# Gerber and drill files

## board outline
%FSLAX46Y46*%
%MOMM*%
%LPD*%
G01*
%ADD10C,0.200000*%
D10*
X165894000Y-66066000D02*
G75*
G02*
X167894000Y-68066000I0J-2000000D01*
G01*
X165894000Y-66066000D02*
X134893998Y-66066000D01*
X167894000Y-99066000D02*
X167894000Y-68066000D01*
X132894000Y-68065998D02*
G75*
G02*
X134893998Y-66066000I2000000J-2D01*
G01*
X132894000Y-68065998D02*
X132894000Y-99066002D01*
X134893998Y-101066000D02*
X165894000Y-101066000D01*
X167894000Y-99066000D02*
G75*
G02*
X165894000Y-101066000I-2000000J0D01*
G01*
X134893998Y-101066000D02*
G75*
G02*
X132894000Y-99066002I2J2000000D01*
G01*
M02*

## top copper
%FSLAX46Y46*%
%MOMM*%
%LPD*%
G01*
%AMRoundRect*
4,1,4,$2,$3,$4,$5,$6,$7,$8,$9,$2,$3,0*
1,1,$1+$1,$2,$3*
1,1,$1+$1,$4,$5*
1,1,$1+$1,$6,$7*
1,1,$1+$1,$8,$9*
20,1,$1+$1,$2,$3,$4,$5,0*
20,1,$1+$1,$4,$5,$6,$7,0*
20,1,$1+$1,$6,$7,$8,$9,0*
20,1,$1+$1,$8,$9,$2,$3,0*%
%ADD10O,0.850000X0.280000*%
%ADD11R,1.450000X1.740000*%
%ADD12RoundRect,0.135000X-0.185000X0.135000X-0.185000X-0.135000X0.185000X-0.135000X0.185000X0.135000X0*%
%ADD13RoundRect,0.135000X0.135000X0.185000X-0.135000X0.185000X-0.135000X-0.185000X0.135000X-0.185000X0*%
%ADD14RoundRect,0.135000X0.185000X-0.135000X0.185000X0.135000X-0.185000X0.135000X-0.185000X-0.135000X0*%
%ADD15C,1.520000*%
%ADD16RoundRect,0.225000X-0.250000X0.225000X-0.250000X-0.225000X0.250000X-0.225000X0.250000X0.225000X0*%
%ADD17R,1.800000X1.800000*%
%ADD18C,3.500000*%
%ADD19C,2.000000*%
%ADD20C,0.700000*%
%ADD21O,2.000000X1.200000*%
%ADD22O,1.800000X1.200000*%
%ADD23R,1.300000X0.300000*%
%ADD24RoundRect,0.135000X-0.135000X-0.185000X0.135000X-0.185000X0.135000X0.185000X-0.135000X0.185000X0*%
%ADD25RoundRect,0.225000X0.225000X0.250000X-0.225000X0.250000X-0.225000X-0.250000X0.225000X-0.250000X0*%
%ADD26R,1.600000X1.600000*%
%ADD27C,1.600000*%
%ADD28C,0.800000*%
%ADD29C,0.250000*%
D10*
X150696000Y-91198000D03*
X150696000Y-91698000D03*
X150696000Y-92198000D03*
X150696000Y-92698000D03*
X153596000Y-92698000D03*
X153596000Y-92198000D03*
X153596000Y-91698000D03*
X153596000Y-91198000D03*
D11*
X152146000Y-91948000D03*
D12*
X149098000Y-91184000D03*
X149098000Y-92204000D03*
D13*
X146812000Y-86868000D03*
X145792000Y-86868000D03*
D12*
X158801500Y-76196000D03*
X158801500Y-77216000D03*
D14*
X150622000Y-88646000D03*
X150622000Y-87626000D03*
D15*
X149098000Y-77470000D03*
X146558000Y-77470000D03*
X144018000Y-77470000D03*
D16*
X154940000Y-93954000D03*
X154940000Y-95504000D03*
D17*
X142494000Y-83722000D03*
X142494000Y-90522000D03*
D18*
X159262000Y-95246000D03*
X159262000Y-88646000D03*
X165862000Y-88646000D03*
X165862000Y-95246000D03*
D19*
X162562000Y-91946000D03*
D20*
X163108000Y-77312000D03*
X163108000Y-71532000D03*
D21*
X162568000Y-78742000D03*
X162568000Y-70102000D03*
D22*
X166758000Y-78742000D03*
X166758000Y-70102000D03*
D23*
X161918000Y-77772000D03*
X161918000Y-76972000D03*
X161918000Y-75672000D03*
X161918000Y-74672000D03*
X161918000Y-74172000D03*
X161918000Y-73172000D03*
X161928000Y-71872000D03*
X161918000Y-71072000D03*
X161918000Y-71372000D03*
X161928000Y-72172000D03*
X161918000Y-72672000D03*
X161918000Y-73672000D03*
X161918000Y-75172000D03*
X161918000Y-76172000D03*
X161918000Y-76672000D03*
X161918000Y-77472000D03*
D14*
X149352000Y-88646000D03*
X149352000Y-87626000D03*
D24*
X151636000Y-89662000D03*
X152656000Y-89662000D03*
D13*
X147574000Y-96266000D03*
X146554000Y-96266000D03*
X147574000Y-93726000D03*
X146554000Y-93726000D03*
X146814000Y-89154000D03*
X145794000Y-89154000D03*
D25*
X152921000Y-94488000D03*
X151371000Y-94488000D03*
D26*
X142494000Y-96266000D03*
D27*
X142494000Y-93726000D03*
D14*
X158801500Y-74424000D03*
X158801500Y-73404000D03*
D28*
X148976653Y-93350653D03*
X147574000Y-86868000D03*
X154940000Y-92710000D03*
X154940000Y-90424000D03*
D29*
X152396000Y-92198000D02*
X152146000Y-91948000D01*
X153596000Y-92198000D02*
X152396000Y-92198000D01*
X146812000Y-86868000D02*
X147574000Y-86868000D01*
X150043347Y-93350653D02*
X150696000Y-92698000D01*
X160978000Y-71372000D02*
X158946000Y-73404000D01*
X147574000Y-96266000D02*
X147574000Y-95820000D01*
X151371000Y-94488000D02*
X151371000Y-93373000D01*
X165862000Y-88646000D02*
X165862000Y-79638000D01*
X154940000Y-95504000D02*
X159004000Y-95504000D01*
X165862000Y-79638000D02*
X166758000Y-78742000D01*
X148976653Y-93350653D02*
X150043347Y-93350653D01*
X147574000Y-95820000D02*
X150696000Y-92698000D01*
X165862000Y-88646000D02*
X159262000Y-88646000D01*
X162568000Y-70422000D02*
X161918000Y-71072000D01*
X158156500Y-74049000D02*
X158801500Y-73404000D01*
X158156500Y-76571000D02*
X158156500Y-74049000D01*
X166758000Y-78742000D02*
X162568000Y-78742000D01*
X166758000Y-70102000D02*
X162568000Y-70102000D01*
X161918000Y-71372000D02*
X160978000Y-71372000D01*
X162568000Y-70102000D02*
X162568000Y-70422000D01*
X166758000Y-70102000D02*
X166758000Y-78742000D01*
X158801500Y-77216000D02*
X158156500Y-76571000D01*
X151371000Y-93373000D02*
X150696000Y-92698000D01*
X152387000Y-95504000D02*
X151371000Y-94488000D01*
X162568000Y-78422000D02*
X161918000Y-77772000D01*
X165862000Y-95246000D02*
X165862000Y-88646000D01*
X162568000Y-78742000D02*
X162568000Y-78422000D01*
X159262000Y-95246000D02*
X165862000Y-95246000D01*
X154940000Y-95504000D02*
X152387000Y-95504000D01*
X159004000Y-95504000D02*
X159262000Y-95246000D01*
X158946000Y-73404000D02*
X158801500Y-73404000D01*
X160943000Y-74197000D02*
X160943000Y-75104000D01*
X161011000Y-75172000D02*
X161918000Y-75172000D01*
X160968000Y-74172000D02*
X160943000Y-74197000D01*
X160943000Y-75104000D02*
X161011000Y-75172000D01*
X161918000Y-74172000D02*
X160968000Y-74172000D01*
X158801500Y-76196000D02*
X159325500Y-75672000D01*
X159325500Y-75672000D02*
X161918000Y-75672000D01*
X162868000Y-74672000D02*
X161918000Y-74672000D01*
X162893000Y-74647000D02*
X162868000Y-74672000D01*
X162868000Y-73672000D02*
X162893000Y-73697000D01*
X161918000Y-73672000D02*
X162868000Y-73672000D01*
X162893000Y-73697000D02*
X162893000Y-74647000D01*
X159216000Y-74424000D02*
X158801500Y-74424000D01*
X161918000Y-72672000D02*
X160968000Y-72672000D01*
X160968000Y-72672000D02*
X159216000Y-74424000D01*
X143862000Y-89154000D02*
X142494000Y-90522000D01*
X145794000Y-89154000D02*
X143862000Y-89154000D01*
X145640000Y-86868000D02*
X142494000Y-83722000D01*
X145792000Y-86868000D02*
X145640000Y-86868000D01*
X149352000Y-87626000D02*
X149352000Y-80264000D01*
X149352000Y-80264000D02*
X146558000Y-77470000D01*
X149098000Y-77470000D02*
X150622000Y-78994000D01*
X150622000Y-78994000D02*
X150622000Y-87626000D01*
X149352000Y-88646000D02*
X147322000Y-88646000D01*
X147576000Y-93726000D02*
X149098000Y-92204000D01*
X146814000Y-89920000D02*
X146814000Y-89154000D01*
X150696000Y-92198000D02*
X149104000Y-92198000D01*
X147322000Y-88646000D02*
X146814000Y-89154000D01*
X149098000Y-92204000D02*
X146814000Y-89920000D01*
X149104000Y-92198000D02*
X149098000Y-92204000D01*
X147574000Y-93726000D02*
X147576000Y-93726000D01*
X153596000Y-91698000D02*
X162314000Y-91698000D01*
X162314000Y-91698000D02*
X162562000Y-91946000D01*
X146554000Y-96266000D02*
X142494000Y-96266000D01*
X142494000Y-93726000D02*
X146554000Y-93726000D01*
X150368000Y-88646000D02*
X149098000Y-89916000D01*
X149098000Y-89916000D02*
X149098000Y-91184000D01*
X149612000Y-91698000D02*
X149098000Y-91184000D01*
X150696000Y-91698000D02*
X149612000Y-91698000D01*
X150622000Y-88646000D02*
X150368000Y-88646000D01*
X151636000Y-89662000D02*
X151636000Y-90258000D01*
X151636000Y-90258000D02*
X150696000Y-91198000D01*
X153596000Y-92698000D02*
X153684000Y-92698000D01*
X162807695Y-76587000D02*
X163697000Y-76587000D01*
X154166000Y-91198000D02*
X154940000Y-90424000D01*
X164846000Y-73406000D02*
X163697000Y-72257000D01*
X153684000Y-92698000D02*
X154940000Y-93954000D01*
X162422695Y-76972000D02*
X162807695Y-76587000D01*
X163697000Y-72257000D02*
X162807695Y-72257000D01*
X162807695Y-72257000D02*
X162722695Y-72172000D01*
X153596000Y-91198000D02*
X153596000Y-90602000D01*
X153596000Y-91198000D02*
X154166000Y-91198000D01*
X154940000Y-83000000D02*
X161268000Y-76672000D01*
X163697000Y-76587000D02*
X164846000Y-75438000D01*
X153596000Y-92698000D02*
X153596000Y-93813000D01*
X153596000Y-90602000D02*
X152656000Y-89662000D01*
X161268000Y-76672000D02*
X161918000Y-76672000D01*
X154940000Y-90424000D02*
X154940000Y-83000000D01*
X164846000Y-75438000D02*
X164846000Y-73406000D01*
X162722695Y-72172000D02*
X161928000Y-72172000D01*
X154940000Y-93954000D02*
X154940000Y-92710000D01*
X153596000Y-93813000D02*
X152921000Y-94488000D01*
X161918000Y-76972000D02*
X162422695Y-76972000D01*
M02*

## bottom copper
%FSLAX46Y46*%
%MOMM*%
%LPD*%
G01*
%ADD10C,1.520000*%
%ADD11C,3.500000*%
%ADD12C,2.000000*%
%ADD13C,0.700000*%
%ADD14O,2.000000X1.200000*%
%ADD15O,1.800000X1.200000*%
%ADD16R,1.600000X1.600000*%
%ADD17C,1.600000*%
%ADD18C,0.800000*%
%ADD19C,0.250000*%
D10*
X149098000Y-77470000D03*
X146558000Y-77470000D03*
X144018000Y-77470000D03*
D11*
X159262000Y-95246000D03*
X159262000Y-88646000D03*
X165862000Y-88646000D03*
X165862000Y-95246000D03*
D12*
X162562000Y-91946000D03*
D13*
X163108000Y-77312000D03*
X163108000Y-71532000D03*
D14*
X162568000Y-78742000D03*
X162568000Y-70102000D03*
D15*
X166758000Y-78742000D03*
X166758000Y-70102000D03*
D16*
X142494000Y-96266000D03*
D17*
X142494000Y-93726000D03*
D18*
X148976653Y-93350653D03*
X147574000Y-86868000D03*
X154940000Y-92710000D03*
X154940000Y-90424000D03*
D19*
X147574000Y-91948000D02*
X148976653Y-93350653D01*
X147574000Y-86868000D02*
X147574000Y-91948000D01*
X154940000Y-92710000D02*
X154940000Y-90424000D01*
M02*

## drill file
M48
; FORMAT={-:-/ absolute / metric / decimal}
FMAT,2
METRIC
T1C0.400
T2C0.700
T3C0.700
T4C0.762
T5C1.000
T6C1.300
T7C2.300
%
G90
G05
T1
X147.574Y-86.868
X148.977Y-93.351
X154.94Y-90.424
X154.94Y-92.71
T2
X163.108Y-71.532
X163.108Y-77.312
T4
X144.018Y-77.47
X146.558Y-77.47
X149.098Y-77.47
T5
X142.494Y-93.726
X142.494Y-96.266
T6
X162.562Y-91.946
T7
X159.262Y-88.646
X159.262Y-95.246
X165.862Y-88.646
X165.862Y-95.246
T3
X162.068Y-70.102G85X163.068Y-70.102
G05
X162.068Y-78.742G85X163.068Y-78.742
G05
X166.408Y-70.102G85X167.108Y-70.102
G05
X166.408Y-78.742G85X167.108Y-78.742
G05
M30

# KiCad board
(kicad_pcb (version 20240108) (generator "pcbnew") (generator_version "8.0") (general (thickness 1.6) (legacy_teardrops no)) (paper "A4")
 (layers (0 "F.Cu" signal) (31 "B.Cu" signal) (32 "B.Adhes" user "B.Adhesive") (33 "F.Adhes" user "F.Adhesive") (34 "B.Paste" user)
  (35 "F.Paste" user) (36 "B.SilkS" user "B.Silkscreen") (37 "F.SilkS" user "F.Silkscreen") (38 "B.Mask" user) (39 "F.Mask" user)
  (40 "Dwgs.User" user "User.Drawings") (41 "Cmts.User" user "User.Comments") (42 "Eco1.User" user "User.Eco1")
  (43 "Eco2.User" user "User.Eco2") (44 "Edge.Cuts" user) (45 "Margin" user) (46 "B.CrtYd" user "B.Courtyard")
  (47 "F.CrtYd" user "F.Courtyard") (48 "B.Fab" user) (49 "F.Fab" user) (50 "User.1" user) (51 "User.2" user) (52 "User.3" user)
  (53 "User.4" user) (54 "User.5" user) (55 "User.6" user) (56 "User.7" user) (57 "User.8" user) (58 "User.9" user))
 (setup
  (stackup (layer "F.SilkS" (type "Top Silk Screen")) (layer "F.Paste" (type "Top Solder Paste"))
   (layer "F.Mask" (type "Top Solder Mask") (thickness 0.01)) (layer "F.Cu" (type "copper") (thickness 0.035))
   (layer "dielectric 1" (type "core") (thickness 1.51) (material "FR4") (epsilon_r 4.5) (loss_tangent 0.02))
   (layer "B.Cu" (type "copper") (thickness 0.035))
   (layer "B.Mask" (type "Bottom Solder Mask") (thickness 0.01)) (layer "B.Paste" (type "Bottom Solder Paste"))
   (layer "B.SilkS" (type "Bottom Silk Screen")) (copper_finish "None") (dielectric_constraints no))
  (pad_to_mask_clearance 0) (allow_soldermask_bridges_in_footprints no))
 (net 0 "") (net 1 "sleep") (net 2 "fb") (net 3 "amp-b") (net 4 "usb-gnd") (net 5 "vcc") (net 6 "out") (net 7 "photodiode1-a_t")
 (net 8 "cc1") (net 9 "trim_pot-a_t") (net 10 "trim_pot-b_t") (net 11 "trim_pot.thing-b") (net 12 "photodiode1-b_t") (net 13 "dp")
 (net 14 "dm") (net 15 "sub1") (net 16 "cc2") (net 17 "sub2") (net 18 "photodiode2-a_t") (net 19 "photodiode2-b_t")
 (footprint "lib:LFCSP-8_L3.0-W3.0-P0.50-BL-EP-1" (layer "F.Cu") (at 152.146 91.948 -90)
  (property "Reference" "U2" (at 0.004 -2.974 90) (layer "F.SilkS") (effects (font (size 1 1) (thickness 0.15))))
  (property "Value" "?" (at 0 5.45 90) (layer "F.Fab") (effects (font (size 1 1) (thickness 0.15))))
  (pad "1" smd oval (at -0.75 1.45 90) (size 0.28 0.85) (layers "F.Cu" "F.Paste" "F.Mask") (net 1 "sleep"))
  (pad "2" smd oval (at -0.25 1.45 90) (size 0.28 0.85) (layers "F.Cu" "F.Paste" "F.Mask") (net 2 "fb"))
  (pad "3" smd oval (at 0.25 1.45 90) (size 0.28 0.85) (layers "F.Cu" "F.Paste" "F.Mask") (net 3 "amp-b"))
  (pad "4" smd oval (at 0.75 1.45 90) (size 0.28 0.85) (layers "F.Cu" "F.Paste" "F.Mask") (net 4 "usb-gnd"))
  (pad "5" smd oval (at 0.75 -1.45 90) (size 0.28 0.85) (layers "F.Cu" "F.Paste" "F.Mask") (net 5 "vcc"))
  (pad "6" smd oval (at 0.25 -1.45 90) (size 0.28 0.85) (layers "F.Cu" "F.Paste" "F.Mask"))
  (pad "7" smd oval (at -0.25 -1.45 90) (size 0.28 0.85) (layers "F.Cu" "F.Paste" "F.Mask") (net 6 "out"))
  (pad "8" smd oval (at -0.75 -1.45 90) (size 0.28 0.85) (layers "F.Cu" "F.Paste" "F.Mask") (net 5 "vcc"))
  (pad "9" smd rect (at 0 0 270) (size 1.74 1.45) (layers "F.Cu" "F.Paste" "F.Mask")))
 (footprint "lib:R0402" (layer "F.Cu") (at 149.098 91.694 -90)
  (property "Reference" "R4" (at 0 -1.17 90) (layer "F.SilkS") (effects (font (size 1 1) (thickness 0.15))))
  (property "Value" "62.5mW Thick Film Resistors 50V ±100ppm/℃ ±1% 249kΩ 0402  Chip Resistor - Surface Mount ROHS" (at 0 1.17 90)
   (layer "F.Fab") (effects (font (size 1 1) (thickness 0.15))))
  (pad "1" smd roundrect (at -0.51 0 270) (size 0.54 0.64) (layers "F.Cu" "F.Paste" "F.Mask") (roundrect_rratio 0.25) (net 2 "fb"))
  (pad "2" smd roundrect (at 0.51 0 270) (size 0.54 0.64) (layers "F.Cu" "F.Paste" "F.Mask") (roundrect_rratio 0.25) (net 3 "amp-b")))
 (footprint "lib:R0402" (layer "F.Cu") (at 146.302 86.868 180)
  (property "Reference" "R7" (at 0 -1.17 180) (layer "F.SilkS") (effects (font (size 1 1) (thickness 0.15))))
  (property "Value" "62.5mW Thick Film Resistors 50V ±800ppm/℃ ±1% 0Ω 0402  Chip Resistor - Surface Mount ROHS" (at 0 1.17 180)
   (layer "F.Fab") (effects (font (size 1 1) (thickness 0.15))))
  (pad "1" smd roundrect (at -0.51 0 180) (size 0.54 0.64) (layers "F.Cu" "F.Paste" "F.Mask") (roundrect_rratio 0.25) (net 4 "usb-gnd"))
  (pad "2" smd roundrect (at 0.51 0 180) (size 0.54 0.64) (layers "F.Cu" "F.Paste" "F.Mask") (roundrect_rratio 0.25)
   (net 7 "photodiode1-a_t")))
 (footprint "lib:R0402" (layer "F.Cu") (at 158.8015 76.706 -90)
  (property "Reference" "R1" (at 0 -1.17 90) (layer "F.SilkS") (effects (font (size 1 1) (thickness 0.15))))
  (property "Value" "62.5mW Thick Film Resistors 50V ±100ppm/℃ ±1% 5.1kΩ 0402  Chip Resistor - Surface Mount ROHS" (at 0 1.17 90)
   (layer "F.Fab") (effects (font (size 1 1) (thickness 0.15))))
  (pad "1" smd roundrect (at -0.51 0 270) (size 0.54 0.64) (layers "F.Cu" "F.Paste" "F.Mask") (roundrect_rratio 0.25) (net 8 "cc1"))
  (pad "2" smd roundrect (at 0.51 0 270) (size 0.54 0.64) (layers "F.Cu" "F.Paste" "F.Mask") (roundrect_rratio 0.25) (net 4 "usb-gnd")))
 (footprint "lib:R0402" (layer "F.Cu") (at 150.622 88.136 90)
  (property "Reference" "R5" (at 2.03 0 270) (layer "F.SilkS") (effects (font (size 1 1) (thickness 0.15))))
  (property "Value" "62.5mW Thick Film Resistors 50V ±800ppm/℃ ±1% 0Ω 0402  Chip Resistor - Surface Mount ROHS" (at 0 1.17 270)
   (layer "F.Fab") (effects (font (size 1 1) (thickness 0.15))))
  (pad "1" smd roundrect (at -0.51 0 90) (size 0.54 0.64) (layers "F.Cu" "F.Paste" "F.Mask") (roundrect_rratio 0.25) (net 2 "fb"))
  (pad "2" smd roundrect (at 0.51 0 90) (size 0.54 0.64) (layers "F.Cu" "F.Paste" "F.Mask") (roundrect_rratio 0.25) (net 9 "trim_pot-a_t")))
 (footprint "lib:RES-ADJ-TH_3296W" (layer "F.Cu") (at 146.558 77.47 -90)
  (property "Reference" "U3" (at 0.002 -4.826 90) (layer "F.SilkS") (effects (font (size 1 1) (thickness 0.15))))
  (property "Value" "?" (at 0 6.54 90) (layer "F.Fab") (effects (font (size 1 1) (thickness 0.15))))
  (pad "1" thru_hole circle (at 0 -2.54 180) (size 1.52 1.52) (drill 0.762) (layers "*.Cu" "*.Mask") (remove_unused_layers no)
   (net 9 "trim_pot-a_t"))
  (pad "2" thru_hole circle (at 0 0 180) (size 1.52 1.52) (drill 0.762) (layers "*.Cu" "*.Mask") (remove_unused_layers no)
   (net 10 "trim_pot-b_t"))
  (pad "3" thru_hole circle (at 0 2.54 180) (size 1.52 1.52) (drill 0.762) (layers "*.Cu" "*.Mask") (remove_unused_layers no)
   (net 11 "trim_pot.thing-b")))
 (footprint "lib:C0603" (layer "F.Cu") (at 154.94 94.729 -90)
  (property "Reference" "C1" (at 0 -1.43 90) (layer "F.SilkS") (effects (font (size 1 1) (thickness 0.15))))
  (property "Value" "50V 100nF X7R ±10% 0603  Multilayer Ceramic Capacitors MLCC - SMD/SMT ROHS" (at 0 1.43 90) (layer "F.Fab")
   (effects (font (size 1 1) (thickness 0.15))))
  (pad "1" smd roundrect (at -0.775 0 270) (size 0.9 0.95) (layers "F.Cu" "F.Paste" "F.Mask") (roundrect_rratio 0.25) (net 5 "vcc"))
  (pad "2" smd roundrect (at 0.775 0 270) (size 0.9 0.95) (layers "F.Cu" "F.Paste" "F.Mask") (roundrect_rratio 0.25) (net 4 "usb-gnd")))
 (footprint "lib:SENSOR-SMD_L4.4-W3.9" (layer "F.Cu") (at 142.494 87.122 -90)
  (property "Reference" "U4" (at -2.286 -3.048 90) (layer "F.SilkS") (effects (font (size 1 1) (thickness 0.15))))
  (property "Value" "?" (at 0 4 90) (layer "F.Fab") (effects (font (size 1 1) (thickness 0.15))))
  (pad "1" smd rect (at -3.4 0 270) (size 1.8 1.8) (layers "F.Cu" "F.Paste" "F.Mask") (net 7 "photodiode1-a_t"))
  (pad "2" smd rect (at 3.4 0 270) (size 1.8 1.8) (layers "F.Cu" "F.Paste" "F.Mask") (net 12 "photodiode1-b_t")))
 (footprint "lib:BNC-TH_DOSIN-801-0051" (layer "F.Cu") (at 162.562 91.946)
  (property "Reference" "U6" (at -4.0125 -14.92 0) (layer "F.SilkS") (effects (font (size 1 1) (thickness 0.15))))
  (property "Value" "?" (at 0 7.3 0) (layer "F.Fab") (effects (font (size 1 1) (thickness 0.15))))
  (pad "1" thru_hole circle (at -3.3 3.3) (size 3.5 3.5) (drill 2.300021) (layers "*.Cu" "*.Mask") (remove_unused_layers no)
   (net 4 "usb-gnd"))
  (pad "2" thru_hole circle (at -3.3 -3.3) (size 3.5 3.5) (drill 2.300021) (layers "*.Cu" "*.Mask") (remove_unused_layers no)
   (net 4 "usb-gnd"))
  (pad "3" thru_hole circle (at 3.3 -3.3) (size 3.5 3.5) (drill 2.300021) (layers "*.Cu" "*.Mask") (remove_unused_layers no)
   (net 4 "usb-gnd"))
  (pad "4" thru_hole circle (at 3.3 3.3) (size 3.5 3.5) (drill 2.300021) (layers "*.Cu" "*.Mask") (remove_unused_layers no)
   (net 4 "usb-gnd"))
  (pad "5" thru_hole circle (at 0 0) (size 2 2) (drill 1.300023) (layers "*.Cu" "*.Mask") (remove_unused_layers no) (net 6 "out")))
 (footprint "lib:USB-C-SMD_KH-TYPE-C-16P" (layer "F.Cu") (at 164.338 74.422 90)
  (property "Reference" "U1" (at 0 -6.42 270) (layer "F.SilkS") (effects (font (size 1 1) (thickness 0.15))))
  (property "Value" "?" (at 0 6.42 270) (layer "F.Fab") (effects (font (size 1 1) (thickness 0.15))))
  (pad "" thru_hole circle (at -2.89 -1.23 90) (size 0.7 0.7) (drill 0.7) (layers "*.Cu" "*.Mask") (remove_unused_layers no))
  (pad "" thru_hole circle (at 2.89 -1.23 90) (size 0.7 0.7) (drill 0.7) (layers "*.Cu" "*.Mask") (remove_unused_layers no))
  (pad "1" thru_hole oval (at -4.32 -1.77 90) (size 1.2 2) (drill oval 0.700024 1.699997) (layers "*.Cu" "*.Mask") (remove_unused_layers no)
   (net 4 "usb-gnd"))
  (pad "2" thru_hole oval (at 4.32 -1.77 90) (size 1.2 2) (drill oval 0.700024 1.699997) (layers "*.Cu" "*.Mask") (remove_unused_layers no)
   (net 4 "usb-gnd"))
  (pad "3" thru_hole oval (at -4.32 2.42 90) (size 1.2 1.8) (drill oval 0.700024 1.399997) (layers "*.Cu" "*.Mask")
   (remove_unused_layers no) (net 4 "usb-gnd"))
  (pad "4" thru_hole oval (at 4.32 2.42 90) (size 1.2 1.8) (drill oval 0.700024 1.399997) (layers "*.Cu" "*.Mask") (remove_unused_layers no)
   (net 4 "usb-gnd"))
  (pad "A1" smd rect (at -3.35 -2.42 90) (size 0.3 1.3) (layers "F.Cu" "F.Paste" "F.Mask") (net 4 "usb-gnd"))
  (pad "A4" smd rect (at -2.55 -2.42 90) (size 0.3 1.3) (layers "F.Cu" "F.Paste" "F.Mask") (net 5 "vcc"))
  (pad "A5" smd rect (at -1.25 -2.42 90) (size 0.3 1.3) (layers "F.Cu" "F.Paste" "F.Mask") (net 8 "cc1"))
  (pad "A6" smd rect (at -0.25 -2.42 90) (size 0.3 1.3) (layers "F.Cu" "F.Paste" "F.Mask") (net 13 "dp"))
  (pad "A7" smd rect (at 0.25 -2.42 90) (size 0.3 1.3) (layers "F.Cu" "F.Paste" "F.Mask") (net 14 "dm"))
  (pad "A8" smd rect (at 1.25 -2.42 90) (size 0.3 1.3) (layers "F.Cu" "F.Paste" "F.Mask") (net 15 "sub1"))
  (pad "A9" smd rect (at 2.55 -2.41 90) (size 0.3 1.3) (layers "F.Cu" "F.Paste" "F.Mask") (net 5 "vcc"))
  (pad "A12" smd rect (at 3.35 -2.42 90) (size 0.3 1.3) (layers "F.Cu" "F.Paste" "F.Mask") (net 4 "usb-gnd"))
  (pad "B1" smd rect (at 3.05 -2.42 90) (size 0.3 1.3) (layers "F.Cu" "F.Paste" "F.Mask") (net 4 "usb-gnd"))
  (pad "B4" smd rect (at 2.25 -2.41 90) (size 0.3 1.3) (layers "F.Cu" "F.Paste" "F.Mask") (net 5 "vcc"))
  (pad "B5" smd rect (at 1.75 -2.42 90) (size 0.3 1.3) (layers "F.Cu" "F.Paste" "F.Mask") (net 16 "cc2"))
  (pad "B6" smd rect (at 0.75 -2.42 90) (size 0.3 1.3) (layers "F.Cu" "F.Paste" "F.Mask") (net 13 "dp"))
  (pad "B7" smd rect (at -0.75 -2.42 90) (size 0.3 1.3) (layers "F.Cu" "F.Paste" "F.Mask") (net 14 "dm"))
  (pad "B8" smd rect (at -1.75 -2.42 90) (size 0.3 1.3) (layers "F.Cu" "F.Paste" "F.Mask") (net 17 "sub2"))
  (pad "B9" smd rect (at -2.25 -2.42 90) (size 0.3 1.3) (layers "F.Cu" "F.Paste" "F.Mask") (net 5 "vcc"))
  (pad "B12" smd rect (at -3.05 -2.42 90) (size 0.3 1.3) (layers "F.Cu" "F.Paste" "F.Mask") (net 4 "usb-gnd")))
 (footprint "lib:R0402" (layer "F.Cu") (at 149.352 88.136 90)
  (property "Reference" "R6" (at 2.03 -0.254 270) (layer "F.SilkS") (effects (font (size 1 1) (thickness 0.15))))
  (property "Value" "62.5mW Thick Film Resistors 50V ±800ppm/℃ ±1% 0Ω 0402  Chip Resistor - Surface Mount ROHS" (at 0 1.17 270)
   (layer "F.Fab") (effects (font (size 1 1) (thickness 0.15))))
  (pad "1" smd roundrect (at -0.51 0 90) (size 0.54 0.64) (layers "F.Cu" "F.Paste" "F.Mask") (roundrect_rratio 0.25) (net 3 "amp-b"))
  (pad "2" smd roundrect (at 0.51 0 90) (size 0.54 0.64) (layers "F.Cu" "F.Paste" "F.Mask") (roundrect_rratio 0.25) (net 10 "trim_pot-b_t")))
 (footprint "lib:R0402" (layer "F.Cu") (at 152.146 89.662)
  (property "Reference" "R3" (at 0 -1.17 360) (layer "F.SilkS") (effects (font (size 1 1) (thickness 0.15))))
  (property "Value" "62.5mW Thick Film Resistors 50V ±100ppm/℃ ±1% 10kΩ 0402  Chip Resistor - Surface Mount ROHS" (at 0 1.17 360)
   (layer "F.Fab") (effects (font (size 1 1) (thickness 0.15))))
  (pad "1" smd roundrect (at -0.51 0) (size 0.54 0.64) (layers "F.Cu" "F.Paste" "F.Mask") (roundrect_rratio 0.25) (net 1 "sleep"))
  (pad "2" smd roundrect (at 0.51 0) (size 0.54 0.64) (layers "F.Cu" "F.Paste" "F.Mask") (roundrect_rratio 0.25) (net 5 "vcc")))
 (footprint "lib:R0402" (layer "F.Cu") (at 147.064 96.266 180)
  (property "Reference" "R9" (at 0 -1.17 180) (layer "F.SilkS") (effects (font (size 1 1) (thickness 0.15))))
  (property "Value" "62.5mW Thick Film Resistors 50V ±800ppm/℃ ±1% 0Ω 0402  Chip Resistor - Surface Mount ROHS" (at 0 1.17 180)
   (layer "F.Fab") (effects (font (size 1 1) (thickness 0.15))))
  (pad "1" smd roundrect (at -0.51 0 180) (size 0.54 0.64) (layers "F.Cu" "F.Paste" "F.Mask") (roundrect_rratio 0.25) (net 4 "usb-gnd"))
  (pad "2" smd roundrect (at 0.51 0 180) (size 0.54 0.64) (layers "F.Cu" "F.Paste" "F.Mask") (roundrect_rratio 0.25)
   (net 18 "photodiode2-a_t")))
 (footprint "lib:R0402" (layer "F.Cu") (at 147.064 93.726 180)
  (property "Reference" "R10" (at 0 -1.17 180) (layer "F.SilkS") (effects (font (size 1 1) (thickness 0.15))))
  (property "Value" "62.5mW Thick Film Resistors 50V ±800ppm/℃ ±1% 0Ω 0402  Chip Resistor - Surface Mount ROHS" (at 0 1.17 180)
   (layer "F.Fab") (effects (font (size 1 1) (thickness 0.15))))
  (pad "1" smd roundrect (at -0.51 0 180) (size 0.54 0.64) (layers "F.Cu" "F.Paste" "F.Mask") (roundrect_rratio 0.25) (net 3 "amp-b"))
  (pad "2" smd roundrect (at 0.51 0 180) (size 0.54 0.64) (layers "F.Cu" "F.Paste" "F.Mask") (roundrect_rratio 0.25)
   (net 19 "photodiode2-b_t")))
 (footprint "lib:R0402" (layer "F.Cu") (at 146.304 89.154 180)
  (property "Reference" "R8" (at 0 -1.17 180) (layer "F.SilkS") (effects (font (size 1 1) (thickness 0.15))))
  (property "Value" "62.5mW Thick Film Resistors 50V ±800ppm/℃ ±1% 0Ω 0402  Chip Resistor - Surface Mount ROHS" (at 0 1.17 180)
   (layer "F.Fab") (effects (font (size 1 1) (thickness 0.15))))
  (pad "1" smd roundrect (at -0.51 0 180) (size 0.54 0.64) (layers "F.Cu" "F.Paste" "F.Mask") (roundrect_rratio 0.25) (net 3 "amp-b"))
  (pad "2" smd roundrect (at 0.51 0 180) (size 0.54 0.64) (layers "F.Cu" "F.Paste" "F.Mask") (roundrect_rratio 0.25)
   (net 12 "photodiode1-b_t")))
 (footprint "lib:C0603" (layer "F.Cu") (at 152.146 94.488 180)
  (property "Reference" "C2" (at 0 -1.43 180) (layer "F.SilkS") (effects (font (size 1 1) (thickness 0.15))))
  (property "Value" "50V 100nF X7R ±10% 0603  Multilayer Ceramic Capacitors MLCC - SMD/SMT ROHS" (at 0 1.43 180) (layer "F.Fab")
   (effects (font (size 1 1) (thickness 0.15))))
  (pad "1" smd roundrect (at -0.775 0 180) (size 0.9 0.95) (layers "F.Cu" "F.Paste" "F.Mask") (roundrect_rratio 0.25) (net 5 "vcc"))
  (pad "2" smd roundrect (at 0.775 0 180) (size 0.9 0.95) (layers "F.Cu" "F.Paste" "F.Mask") (roundrect_rratio 0.25) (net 4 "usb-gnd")))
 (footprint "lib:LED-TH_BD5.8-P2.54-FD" (layer "F.Cu") (at 142.494 94.996 90)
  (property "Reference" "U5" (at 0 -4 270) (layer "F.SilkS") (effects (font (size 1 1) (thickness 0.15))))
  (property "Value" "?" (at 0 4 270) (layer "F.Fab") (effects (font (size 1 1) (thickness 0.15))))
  (pad "1" thru_hole rect (at -1.27 0 90) (size 1.6 1.6) (drill 0.999998) (layers "*.Cu" "*.Mask") (remove_unused_layers no)
   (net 18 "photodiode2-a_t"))
  (pad "2" thru_hole circle (at 1.27 0 90) (size 1.6 1.6) (drill 0.999998) (layers "*.Cu" "*.Mask") (remove_unused_layers no)
   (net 19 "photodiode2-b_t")))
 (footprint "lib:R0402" (layer "F.Cu") (at 158.8015 73.914 90)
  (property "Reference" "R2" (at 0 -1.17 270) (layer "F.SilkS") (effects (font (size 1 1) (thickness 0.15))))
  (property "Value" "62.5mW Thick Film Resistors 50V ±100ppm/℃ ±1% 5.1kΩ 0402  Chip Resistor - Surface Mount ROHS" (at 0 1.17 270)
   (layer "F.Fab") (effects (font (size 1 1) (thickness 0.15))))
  (pad "1" smd roundrect (at -0.51 0 90) (size 0.54 0.64) (layers "F.Cu" "F.Paste" "F.Mask") (roundrect_rratio 0.25) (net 16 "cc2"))
  (pad "2" smd roundrect (at 0.51 0 90) (size 0.54 0.64) (layers "F.Cu" "F.Paste" "F.Mask") (roundrect_rratio 0.25) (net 4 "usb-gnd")))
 (gr_arc (start 165.894 66.066) (mid 167.308214 66.651786) (end 167.894 68.066) (stroke (width 0.2) (type default)) (layer "Edge.Cuts"))
 (gr_line (start 165.894 66.066) (end 134.893998 66.066) (stroke (width 0.2) (type default)) (layer "Edge.Cuts"))
 (gr_line (start 167.894 99.066) (end 167.894 68.066) (stroke (width 0.2) (type default)) (layer "Edge.Cuts"))
 (gr_arc (start 132.894 68.065998) (mid 133.479786 66.651786) (end 134.893998 66.066) (stroke (width 0.2) (type default))
  (layer "Edge.Cuts"))
 (gr_line (start 132.894 68.065998) (end 132.894 99.066002) (stroke (width 0.2) (type default)) (layer "Edge.Cuts"))
 (gr_line (start 134.893998 101.066) (end 165.894 101.066) (stroke (width 0.2) (type default)) (layer "Edge.Cuts"))
 (gr_arc (start 167.894 99.066) (mid 167.308214 100.480214) (end 165.894 101.066) (stroke (width 0.2) (type default)) (layer "Edge.Cuts"))
 (gr_arc (start 134.893998 101.066) (mid 133.479786 100.480214) (end 132.894 99.066002) (stroke (width 0.2) (type default))
  (layer "Edge.Cuts"))
 (segment (start 152.396 92.198) (end 152.146 91.948) (width 0.25) (layer "F.Cu") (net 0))
 (segment (start 153.596 92.198) (end 152.396 92.198) (width 0.25) (layer "F.Cu") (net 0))
 (segment (start 146.812 86.868) (end 147.574 86.868) (width 0.25) (layer "F.Cu") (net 4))
 (segment (start 150.043347 93.350653) (end 150.696 92.698) (width 0.25) (layer "F.Cu") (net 4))
 (segment (start 160.978 71.372) (end 158.946 73.404) (width 0.25) (layer "F.Cu") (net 4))
 (segment (start 147.574 96.266) (end 147.574 95.82) (width 0.25) (layer "F.Cu") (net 4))
 (segment (start 151.371 94.488) (end 151.371 93.373) (width 0.25) (layer "F.Cu") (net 4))
 (segment (start 165.862 88.646) (end 165.862 79.638) (width 0.25) (layer "F.Cu") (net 4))
 (segment (start 154.94 95.504) (end 159.004 95.504) (width 0.25) (layer "F.Cu") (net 4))
 (segment (start 165.862 79.638) (end 166.758 78.742) (width 0.25) (layer "F.Cu") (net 4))
 (segment (start 148.976653 93.350653) (end 150.043347 93.350653) (width 0.25) (layer "F.Cu") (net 4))
 (segment (start 147.574 95.82) (end 150.696 92.698) (width 0.25) (layer "F.Cu") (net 4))
 (segment (start 165.862 88.646) (end 159.262 88.646) (width 0.25) (layer "F.Cu") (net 4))
 (segment (start 162.568 70.422) (end 161.918 71.072) (width 0.25) (layer "F.Cu") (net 4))
 (segment (start 158.1565 74.049) (end 158.8015 73.404) (width 0.25) (layer "F.Cu") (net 4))
 (segment (start 158.1565 76.571) (end 158.1565 74.049) (width 0.25) (layer "F.Cu") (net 4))
 (segment (start 166.758 78.742) (end 162.568 78.742) (width 0.25) (layer "F.Cu") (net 4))
 (segment (start 166.758 70.102) (end 162.568 70.102) (width 0.25) (layer "F.Cu") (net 4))
 (segment (start 161.918 71.372) (end 160.978 71.372) (width 0.25) (layer "F.Cu") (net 4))
 (segment (start 162.568 70.102) (end 162.568 70.422) (width 0.25) (layer "F.Cu") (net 4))
 (segment (start 166.758 70.102) (end 166.758 78.742) (width 0.25) (layer "F.Cu") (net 4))
 (segment (start 158.8015 77.216) (end 158.1565 76.571) (width 0.25) (layer "F.Cu") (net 4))
 (segment (start 151.371 93.373) (end 150.696 92.698) (width 0.25) (layer "F.Cu") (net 4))
 (segment (start 152.387 95.504) (end 151.371 94.488) (width 0.25) (layer "F.Cu") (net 4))
 (segment (start 162.568 78.422) (end 161.918 77.772) (width 0.25) (layer "F.Cu") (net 4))
 (segment (start 165.862 95.246) (end 165.862 88.646) (width 0.25) (layer "F.Cu") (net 4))
 (segment (start 162.568 78.742) (end 162.568 78.422) (width 0.25) (layer "F.Cu") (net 4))
 (segment (start 159.262 95.246) (end 165.862 95.246) (width 0.25) (layer "F.Cu") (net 4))
 (segment (start 154.94 95.504) (end 152.387 95.504) (width 0.25) (layer "F.Cu") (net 4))
 (segment (start 159.004 95.504) (end 159.262 95.246) (width 0.25) (layer "F.Cu") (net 4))
 (segment (start 158.946 73.404) (end 158.8015 73.404) (width 0.25) (layer "F.Cu") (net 4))
 (via (at 148.976653 93.350653) (size 0.8) (drill 0.4) (layers "F.Cu" "B.Cu") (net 4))
 (via (at 147.574 86.868) (size 0.8) (drill 0.4) (layers "F.Cu" "B.Cu") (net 4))
 (segment (start 147.574 91.948) (end 148.976653 93.350653) (width 0.25) (layer "B.Cu") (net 4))
 (segment (start 147.574 86.868) (end 147.574 91.948) (width 0.25) (layer "B.Cu") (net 4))
 (segment (start 160.943 74.197) (end 160.943 75.104) (width 0.25) (layer "F.Cu") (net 14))
 (segment (start 161.011 75.172) (end 161.918 75.172) (width 0.25) (layer "F.Cu") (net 14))
 (segment (start 160.968 74.172) (end 160.943 74.197) (width 0.25) (layer "F.Cu") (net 14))
 (segment (start 160.943 75.104) (end 161.011 75.172) (width 0.25) (layer "F.Cu") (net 14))
 (segment (start 161.918 74.172) (end 160.968 74.172) (width 0.25) (layer "F.Cu") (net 14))
 (segment (start 158.8015 76.196) (end 159.3255 75.672) (width 0.25) (layer "F.Cu") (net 8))
 (segment (start 159.3255 75.672) (end 161.918 75.672) (width 0.25) (layer "F.Cu") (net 8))
 (segment (start 162.868 74.672) (end 161.918 74.672) (width 0.25) (layer "F.Cu") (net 13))
 (segment (start 162.893 74.647) (end 162.868 74.672) (width 0.25) (layer "F.Cu") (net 13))
 (segment (start 162.868 73.672) (end 162.893 73.697) (width 0.25) (layer "F.Cu") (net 13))
 (segment (start 161.918 73.672) (end 162.868 73.672) (width 0.25) (layer "F.Cu") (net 13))
 (segment (start 162.893 73.697) (end 162.893 74.647) (width 0.25) (layer "F.Cu") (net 13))
 (segment (start 159.216 74.424) (end 158.8015 74.424) (width 0.25) (layer "F.Cu") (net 16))
 (segment (start 161.918 72.672) (end 160.968 72.672) (width 0.25) (layer "F.Cu") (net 16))
 (segment (start 160.968 72.672) (end 159.216 74.424) (width 0.25) (layer "F.Cu") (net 16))
 (segment (start 143.862 89.154) (end 142.494 90.522) (width 0.25) (layer "F.Cu") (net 12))
 (segment (start 145.794 89.154) (end 143.862 89.154) (width 0.25) (layer "F.Cu") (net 12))
 (segment (start 145.64 86.868) (end 142.494 83.722) (width 0.25) (layer "F.Cu") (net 7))
 (segment (start 145.792 86.868) (end 145.64 86.868) (width 0.25) (layer "F.Cu") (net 7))
 (segment (start 149.352 87.626) (end 149.352 80.264) (width 0.25) (layer "F.Cu") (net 10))
 (segment (start 149.352 80.264) (end 146.558 77.47) (width 0.25) (layer "F.Cu") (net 10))
 (segment (start 149.098 77.47) (end 150.622 78.994) (width 0.25) (layer "F.Cu") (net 9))
 (segment (start 150.622 78.994) (end 150.622 87.626) (width 0.25) (layer "F.Cu") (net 9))
 (segment (start 149.352 88.646) (end 147.322 88.646) (width 0.25) (layer "F.Cu") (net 3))
 (segment (start 147.576 93.726) (end 149.098 92.204) (width 0.25) (layer "F.Cu") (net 3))
 (segment (start 146.814 89.92) (end 146.814 89.154) (width 0.25) (layer "F.Cu") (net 3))
 (segment (start 150.696 92.198) (end 149.104 92.198) (width 0.25) (layer "F.Cu") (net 3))
 (segment (start 147.322 88.646) (end 146.814 89.154) (width 0.25) (layer "F.Cu") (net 3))
 (segment (start 149.098 92.204) (end 146.814 89.92) (width 0.25) (layer "F.Cu") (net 3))
 (segment (start 149.104 92.198) (end 149.098 92.204) (width 0.25) (layer "F.Cu") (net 3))
 (segment (start 147.574 93.726) (end 147.576 93.726) (width 0.25) (layer "F.Cu") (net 3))
 (segment (start 153.596 91.698) (end 162.314 91.698) (width 0.25) (layer "F.Cu") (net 6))
 (segment (start 162.314 91.698) (end 162.562 91.946) (width 0.25) (layer "F.Cu") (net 6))
 (segment (start 146.554 96.266) (end 142.494 96.266) (width 0.25) (layer "F.Cu") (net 18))
 (segment (start 142.494 93.726) (end 146.554 93.726) (width 0.25) (layer "F.Cu") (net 19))
 (segment (start 150.368 88.646) (end 149.098 89.916) (width 0.25) (layer "F.Cu") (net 2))
 (segment (start 149.098 89.916) (end 149.098 91.184) (width 0.25) (layer "F.Cu") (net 2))
 (segment (start 149.612 91.698) (end 149.098 91.184) (width 0.25) (layer "F.Cu") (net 2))
 (segment (start 150.696 91.698) (end 149.612 91.698) (width 0.25) (layer "F.Cu") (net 2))
 (segment (start 150.622 88.646) (end 150.368 88.646) (width 0.25) (layer "F.Cu") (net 2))
 (segment (start 151.636 89.662) (end 151.636 90.258) (width 0.25) (layer "F.Cu") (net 1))
 (segment (start 151.636 90.258) (end 150.696 91.198) (width 0.25) (layer "F.Cu") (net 1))
 (segment (start 153.596 92.698) (end 153.684 92.698) (width 0.25) (layer "F.Cu") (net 5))
 (segment (start 162.807695 76.587) (end 163.697 76.587) (width 0.25) (layer "F.Cu") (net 5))
 (segment (start 154.166 91.198) (end 154.94 90.424) (width 0.25) (layer "F.Cu") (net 5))
 (segment (start 164.846 73.406) (end 163.697 72.257) (width 0.25) (layer "F.Cu") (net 5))
 (segment (start 153.684 92.698) (end 154.94 93.954) (width 0.25) (layer "F.Cu") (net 5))
 (segment (start 162.422695 76.972) (end 162.807695 76.587) (width 0.25) (layer "F.Cu") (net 5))
 (segment (start 163.697 72.257) (end 162.807695 72.257) (width 0.25) (layer "F.Cu") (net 5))
 (segment (start 162.807695 72.257) (end 162.722695 72.172) (width 0.25) (layer "F.Cu") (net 5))
 (segment (start 153.596 91.198) (end 153.596 90.602) (width 0.25) (layer "F.Cu") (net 5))
 (segment (start 153.596 91.198) (end 154.166 91.198) (width 0.25) (layer "F.Cu") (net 5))
 (segment (start 154.94 83) (end 161.268 76.672) (width 0.25) (layer "F.Cu") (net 5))
 (segment (start 163.697 76.587) (end 164.846 75.438) (width 0.25) (layer "F.Cu") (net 5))
 (segment (start 153.596 92.698) (end 153.596 93.813) (width 0.25) (layer "F.Cu") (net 5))
 (segment (start 153.596 90.602) (end 152.656 89.662) (width 0.25) (layer "F.Cu") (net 5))
 (segment (start 161.268 76.672) (end 161.918 76.672) (width 0.25) (layer "F.Cu") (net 5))
 (segment (start 154.94 90.424) (end 154.94 83) (width 0.25) (layer "F.Cu") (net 5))
 (segment (start 164.846 75.438) (end 164.846 73.406) (width 0.25) (layer "F.Cu") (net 5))
 (segment (start 162.722695 72.172) (end 161.928 72.172) (width 0.25) (layer "F.Cu") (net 5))
 (segment (start 154.94 93.954) (end 154.94 92.71) (width 0.25) (layer "F.Cu") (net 5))
 (segment (start 153.596 93.813) (end 152.921 94.488) (width 0.25) (layer "F.Cu") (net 5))
 (segment (start 161.918 76.972) (end 162.422695 76.972) (width 0.25) (layer "F.Cu") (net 5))
 (via (at 154.94 92.71) (size 0.8) (drill 0.4) (layers "F.Cu" "B.Cu") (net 5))
 (via (at 154.94 90.424) (size 0.8) (drill 0.4) (layers "F.Cu" "B.Cu") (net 5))
 (segment (start 154.94 92.71) (end 154.94 90.424) (width 0.25) (layer "B.Cu") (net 5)))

